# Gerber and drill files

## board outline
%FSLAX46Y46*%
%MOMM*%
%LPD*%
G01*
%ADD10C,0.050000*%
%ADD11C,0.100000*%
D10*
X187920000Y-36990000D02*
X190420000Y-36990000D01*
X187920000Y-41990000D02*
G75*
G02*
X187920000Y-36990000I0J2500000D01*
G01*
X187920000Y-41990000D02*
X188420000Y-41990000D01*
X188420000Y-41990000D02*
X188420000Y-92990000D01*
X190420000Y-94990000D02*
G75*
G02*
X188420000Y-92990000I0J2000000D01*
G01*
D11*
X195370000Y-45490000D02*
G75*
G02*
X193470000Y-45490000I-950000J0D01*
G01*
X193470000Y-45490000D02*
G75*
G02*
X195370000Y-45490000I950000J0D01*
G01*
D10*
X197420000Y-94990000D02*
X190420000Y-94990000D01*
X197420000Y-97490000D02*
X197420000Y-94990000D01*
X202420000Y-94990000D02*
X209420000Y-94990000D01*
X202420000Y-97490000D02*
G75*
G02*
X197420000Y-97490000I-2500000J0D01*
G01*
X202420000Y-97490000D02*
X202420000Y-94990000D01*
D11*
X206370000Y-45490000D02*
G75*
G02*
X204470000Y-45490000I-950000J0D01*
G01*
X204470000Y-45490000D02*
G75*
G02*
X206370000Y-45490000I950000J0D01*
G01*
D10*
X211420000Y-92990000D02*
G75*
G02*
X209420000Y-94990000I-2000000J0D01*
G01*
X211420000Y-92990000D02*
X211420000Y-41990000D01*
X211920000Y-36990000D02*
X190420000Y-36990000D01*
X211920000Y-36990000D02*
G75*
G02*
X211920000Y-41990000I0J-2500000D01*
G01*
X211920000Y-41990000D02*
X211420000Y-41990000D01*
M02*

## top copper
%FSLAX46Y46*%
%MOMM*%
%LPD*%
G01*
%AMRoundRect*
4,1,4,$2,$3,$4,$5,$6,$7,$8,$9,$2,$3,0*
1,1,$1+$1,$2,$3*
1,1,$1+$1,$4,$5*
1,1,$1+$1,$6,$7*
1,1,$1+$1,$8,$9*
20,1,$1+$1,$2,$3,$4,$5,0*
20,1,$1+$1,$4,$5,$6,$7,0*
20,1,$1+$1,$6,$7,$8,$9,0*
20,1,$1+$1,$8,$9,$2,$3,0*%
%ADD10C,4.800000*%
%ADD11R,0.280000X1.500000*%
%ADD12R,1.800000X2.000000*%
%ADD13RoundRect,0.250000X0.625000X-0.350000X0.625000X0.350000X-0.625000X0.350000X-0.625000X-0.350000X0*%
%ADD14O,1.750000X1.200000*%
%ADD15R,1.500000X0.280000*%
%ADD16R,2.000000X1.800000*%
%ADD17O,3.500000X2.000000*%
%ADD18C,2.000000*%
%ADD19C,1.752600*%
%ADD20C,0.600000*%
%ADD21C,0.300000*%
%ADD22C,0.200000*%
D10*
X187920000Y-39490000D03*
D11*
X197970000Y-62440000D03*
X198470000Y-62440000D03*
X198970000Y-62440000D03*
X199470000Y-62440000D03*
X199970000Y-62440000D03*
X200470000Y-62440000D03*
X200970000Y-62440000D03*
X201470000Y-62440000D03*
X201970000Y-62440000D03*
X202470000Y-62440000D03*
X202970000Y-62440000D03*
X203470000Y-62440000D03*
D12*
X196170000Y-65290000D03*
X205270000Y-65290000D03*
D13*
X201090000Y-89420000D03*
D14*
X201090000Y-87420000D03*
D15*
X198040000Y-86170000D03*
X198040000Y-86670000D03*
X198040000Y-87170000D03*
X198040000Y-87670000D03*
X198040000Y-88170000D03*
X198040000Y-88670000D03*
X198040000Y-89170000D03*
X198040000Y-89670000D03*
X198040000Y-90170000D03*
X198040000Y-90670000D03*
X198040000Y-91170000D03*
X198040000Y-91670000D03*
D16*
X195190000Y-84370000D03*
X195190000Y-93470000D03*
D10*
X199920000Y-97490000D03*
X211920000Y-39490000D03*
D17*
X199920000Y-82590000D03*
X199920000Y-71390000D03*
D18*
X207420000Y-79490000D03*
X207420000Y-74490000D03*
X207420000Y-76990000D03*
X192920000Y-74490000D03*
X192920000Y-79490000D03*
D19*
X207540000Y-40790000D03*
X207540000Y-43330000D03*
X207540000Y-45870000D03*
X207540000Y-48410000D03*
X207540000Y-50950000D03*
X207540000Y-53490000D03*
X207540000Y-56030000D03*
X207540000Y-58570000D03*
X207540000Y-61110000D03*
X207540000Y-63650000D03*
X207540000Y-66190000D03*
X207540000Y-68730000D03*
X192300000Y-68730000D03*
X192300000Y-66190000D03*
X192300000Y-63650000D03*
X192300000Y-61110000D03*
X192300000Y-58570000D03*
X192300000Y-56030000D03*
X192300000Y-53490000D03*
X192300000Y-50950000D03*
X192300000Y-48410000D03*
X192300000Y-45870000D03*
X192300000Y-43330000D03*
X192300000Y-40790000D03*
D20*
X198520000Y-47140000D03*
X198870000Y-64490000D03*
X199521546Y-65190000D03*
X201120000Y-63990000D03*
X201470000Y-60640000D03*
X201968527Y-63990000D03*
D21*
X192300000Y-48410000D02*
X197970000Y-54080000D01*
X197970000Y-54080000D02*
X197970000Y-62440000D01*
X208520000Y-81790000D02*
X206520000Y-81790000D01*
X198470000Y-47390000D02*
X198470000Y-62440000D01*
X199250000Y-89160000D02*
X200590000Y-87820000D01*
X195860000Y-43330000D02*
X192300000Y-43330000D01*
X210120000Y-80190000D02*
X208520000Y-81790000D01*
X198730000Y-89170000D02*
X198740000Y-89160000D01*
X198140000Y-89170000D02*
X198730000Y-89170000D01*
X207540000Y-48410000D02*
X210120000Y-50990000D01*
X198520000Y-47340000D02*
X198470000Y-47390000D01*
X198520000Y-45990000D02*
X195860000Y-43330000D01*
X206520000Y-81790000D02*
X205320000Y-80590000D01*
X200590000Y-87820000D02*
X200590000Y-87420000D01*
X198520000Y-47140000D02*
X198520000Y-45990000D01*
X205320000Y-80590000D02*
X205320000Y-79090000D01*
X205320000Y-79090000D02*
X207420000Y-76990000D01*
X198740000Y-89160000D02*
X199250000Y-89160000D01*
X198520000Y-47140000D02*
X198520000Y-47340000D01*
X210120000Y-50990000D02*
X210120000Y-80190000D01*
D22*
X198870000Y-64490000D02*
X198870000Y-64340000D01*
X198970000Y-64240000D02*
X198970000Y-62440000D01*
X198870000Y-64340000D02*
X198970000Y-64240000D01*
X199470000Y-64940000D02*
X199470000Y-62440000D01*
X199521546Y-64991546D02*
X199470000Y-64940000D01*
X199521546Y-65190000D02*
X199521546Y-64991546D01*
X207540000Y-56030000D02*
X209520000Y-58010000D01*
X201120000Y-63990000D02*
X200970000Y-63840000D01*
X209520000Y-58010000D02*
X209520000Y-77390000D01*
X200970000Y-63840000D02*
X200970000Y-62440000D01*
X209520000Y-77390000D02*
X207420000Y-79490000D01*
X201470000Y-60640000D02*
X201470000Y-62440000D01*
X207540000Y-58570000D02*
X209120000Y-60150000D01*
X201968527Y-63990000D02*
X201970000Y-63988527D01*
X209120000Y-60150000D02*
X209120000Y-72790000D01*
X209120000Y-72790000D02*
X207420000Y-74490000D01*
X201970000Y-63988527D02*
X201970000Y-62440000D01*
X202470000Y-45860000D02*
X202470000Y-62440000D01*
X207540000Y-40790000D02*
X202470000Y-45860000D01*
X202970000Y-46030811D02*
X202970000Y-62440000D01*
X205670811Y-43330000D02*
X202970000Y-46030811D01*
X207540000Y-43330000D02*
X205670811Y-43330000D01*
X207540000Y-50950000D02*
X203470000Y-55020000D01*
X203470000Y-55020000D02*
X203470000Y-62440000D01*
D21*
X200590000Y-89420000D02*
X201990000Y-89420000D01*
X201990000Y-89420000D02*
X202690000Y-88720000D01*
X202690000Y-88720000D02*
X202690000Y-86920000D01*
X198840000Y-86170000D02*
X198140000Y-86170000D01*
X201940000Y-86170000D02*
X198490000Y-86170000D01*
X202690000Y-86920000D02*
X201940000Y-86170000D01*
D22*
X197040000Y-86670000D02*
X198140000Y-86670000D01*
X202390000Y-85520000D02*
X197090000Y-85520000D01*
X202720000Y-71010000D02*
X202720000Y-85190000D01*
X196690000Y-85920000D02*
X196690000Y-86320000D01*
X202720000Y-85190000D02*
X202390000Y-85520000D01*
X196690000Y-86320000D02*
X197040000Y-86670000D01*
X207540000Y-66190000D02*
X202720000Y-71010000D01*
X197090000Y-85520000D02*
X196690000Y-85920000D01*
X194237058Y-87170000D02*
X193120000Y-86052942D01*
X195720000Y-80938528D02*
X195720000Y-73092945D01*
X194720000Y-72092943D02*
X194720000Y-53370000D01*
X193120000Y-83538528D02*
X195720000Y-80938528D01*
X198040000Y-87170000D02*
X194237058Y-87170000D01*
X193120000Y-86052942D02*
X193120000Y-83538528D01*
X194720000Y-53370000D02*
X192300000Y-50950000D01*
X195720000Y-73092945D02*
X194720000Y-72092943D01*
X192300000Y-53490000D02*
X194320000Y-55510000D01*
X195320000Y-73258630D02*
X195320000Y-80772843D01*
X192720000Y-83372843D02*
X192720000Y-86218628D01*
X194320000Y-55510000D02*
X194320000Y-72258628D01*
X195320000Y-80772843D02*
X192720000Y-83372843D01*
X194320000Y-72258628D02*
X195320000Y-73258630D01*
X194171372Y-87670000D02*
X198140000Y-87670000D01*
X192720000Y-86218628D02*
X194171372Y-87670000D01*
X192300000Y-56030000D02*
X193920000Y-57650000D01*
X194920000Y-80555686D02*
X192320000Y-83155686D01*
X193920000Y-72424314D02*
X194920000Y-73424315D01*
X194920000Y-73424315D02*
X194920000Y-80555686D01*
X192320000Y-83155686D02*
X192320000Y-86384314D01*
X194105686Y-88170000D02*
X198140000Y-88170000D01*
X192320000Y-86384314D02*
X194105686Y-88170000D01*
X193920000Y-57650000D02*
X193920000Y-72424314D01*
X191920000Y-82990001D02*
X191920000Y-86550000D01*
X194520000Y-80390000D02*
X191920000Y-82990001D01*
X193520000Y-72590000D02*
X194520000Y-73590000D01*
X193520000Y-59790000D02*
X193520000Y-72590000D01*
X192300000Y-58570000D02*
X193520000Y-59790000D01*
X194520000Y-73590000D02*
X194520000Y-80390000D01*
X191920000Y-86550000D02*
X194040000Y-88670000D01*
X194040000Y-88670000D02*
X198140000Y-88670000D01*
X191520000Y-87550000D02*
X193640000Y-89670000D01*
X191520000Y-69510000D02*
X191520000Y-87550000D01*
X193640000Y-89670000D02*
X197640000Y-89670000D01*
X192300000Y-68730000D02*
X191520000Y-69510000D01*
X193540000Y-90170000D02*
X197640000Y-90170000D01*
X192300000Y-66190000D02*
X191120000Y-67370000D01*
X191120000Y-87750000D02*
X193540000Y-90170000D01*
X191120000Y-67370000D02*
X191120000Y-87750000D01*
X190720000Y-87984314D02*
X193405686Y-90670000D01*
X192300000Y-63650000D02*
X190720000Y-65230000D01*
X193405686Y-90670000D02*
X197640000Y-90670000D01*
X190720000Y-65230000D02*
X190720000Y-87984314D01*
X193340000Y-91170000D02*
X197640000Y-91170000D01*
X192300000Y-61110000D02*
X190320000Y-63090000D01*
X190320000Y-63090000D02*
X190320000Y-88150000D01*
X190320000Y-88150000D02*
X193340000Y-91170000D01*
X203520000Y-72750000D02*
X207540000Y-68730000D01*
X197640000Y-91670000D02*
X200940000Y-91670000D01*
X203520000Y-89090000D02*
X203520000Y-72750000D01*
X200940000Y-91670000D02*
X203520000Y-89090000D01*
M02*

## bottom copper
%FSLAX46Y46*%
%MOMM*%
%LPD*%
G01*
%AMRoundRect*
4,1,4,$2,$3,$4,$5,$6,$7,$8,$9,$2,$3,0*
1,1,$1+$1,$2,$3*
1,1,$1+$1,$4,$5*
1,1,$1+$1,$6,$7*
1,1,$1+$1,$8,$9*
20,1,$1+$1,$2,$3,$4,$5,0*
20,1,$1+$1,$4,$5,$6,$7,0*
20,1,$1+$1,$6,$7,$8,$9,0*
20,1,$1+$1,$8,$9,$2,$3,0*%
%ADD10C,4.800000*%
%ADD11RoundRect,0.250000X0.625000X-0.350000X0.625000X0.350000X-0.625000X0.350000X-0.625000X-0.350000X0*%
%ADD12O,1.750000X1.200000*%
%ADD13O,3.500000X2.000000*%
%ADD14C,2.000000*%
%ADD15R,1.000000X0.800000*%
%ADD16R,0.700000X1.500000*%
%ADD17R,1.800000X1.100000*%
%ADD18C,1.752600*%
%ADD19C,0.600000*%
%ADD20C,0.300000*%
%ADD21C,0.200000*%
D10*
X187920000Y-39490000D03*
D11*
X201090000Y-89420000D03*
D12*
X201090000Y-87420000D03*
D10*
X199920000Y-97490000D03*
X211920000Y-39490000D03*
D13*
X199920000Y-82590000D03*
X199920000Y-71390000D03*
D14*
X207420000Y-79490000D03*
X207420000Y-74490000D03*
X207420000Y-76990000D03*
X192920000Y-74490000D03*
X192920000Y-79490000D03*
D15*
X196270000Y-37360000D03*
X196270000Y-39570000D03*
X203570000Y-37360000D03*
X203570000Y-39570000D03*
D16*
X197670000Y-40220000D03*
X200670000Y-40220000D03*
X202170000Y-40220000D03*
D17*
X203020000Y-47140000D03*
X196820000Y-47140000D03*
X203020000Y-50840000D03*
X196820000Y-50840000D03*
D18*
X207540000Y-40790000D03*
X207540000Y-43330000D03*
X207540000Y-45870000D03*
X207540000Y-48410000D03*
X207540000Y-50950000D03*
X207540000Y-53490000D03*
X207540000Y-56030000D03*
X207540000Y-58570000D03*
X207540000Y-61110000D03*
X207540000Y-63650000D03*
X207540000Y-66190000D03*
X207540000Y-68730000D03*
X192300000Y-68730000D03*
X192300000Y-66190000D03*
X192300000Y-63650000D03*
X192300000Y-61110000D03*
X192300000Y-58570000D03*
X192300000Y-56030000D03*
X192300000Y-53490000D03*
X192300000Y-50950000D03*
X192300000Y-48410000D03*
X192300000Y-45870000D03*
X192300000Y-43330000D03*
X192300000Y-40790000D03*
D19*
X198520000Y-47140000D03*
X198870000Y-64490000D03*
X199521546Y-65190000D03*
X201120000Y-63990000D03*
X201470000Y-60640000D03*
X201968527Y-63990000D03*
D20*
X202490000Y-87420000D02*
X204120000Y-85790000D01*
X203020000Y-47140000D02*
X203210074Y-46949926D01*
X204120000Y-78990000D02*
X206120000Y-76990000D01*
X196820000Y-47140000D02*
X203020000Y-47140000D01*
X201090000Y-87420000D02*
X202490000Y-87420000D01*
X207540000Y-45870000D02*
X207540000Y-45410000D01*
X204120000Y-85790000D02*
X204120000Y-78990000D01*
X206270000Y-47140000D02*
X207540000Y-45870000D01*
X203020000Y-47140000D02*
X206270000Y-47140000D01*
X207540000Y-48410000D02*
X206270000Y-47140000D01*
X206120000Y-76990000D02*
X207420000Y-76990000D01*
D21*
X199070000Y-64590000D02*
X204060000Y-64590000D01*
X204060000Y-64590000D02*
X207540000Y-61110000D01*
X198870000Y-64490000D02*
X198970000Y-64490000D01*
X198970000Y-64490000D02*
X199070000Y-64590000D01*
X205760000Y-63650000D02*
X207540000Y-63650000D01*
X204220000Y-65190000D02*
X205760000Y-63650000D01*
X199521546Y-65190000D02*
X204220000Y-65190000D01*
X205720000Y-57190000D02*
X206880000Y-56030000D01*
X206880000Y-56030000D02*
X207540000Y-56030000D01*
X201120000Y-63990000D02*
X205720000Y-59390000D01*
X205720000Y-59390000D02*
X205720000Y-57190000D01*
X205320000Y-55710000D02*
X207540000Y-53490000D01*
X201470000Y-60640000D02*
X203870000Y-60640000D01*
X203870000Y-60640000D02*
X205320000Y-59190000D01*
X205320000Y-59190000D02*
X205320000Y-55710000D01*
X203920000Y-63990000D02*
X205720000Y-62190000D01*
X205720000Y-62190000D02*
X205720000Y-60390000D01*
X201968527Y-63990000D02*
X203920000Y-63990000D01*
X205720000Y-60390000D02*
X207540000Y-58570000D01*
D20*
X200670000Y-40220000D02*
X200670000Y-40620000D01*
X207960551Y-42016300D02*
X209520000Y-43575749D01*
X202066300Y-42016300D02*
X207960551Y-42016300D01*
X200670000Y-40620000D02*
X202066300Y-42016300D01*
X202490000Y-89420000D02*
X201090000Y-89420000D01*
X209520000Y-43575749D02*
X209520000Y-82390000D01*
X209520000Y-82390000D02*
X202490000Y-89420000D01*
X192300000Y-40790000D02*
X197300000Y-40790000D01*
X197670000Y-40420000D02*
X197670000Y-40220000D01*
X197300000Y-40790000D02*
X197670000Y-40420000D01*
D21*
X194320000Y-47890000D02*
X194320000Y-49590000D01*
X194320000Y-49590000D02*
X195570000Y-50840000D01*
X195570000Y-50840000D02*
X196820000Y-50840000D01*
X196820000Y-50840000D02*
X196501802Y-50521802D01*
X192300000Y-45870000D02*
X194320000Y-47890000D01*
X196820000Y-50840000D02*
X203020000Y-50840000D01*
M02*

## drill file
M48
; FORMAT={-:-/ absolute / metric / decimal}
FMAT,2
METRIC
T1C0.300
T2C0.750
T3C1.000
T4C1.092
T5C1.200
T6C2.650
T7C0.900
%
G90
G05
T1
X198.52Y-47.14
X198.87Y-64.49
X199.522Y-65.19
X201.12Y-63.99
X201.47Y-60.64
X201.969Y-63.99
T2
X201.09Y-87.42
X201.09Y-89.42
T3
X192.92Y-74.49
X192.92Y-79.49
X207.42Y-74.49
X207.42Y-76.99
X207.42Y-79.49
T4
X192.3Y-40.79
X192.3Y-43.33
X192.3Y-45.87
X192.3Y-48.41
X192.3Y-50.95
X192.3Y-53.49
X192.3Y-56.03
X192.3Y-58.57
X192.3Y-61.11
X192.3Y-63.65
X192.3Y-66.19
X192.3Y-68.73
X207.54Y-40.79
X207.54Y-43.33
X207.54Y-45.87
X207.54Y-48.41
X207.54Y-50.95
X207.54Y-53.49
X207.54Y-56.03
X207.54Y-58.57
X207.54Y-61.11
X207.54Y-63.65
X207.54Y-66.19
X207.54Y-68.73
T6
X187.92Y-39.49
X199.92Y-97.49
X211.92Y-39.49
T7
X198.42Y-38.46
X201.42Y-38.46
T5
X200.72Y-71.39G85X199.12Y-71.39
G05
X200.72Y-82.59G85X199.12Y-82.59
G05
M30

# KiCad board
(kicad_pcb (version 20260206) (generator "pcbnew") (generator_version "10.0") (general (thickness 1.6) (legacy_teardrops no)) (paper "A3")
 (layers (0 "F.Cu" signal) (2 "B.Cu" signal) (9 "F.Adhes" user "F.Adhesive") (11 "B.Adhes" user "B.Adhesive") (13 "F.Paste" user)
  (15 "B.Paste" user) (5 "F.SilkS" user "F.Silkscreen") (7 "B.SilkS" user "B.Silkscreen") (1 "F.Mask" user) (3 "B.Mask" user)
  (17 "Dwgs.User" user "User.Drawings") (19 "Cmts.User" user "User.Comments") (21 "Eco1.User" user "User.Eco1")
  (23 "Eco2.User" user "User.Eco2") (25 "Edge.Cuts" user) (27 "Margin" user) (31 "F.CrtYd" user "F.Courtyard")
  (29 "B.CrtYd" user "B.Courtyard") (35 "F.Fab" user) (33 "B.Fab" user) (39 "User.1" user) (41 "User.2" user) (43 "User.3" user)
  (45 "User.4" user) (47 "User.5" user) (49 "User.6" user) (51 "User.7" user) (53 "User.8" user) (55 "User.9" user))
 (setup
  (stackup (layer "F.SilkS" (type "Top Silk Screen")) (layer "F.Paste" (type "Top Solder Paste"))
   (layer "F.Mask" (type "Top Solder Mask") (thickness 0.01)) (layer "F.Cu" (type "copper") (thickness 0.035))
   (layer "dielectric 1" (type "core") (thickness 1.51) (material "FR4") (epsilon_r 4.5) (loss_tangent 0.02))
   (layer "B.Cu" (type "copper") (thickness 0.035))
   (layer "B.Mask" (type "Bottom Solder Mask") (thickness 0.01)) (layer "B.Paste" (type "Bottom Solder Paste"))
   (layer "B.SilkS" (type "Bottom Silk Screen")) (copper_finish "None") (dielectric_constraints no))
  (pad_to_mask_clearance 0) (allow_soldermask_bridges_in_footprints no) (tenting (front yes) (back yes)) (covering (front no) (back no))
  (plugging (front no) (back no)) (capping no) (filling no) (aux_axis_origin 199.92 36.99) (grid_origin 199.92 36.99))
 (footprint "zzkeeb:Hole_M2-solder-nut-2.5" (layer "F.Cu") (at 187.92 39.49)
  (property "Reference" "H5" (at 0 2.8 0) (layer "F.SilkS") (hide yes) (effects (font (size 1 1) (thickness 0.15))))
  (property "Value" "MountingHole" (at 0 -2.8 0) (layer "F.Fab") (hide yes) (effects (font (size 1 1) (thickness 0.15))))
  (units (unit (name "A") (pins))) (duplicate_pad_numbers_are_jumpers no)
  (pad "" thru_hole circle (at 0 0) (size 4.8 4.8) (drill 2.65) (layers "*.Cu" "F.Mask") (remove_unused_layers no)))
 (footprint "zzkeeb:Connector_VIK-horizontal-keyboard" (layer "F.Cu") (at 200.72 63.99)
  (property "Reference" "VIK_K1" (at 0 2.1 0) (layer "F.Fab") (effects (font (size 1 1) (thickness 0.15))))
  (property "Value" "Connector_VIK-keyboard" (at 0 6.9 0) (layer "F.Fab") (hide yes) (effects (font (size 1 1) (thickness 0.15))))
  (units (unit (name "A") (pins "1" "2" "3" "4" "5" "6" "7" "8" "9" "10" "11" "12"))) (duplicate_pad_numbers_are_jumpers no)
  (pad "1" smd rect (at -2.75 -1.55) (size 0.28 1.5) (layers "F.Cu" "F.Mask" "F.Paste") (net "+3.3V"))
  (pad "2" smd rect (at -2.25 -1.55) (size 0.28 1.5) (layers "F.Cu" "F.Mask" "F.Paste") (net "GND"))
  (pad "3" smd rect (at -1.75 -1.55) (size 0.28 1.5) (layers "F.Cu" "F.Mask" "F.Paste") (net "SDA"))
  (pad "4" smd rect (at -1.25 -1.55) (size 0.28 1.5) (layers "F.Cu" "F.Mask" "F.Paste") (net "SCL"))
  (pad "5" smd rect (at -0.75 -1.55) (size 0.28 1.5) (layers "F.Cu" "F.Mask" "F.Paste") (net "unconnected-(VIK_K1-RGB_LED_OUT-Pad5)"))
  (pad "6" smd rect (at -0.25 -1.55) (size 0.28 1.5) (layers "F.Cu" "F.Mask" "F.Paste") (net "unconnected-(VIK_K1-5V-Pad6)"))
  (pad "7" smd rect (at 0.25 -1.55) (size 0.28 1.5) (layers "F.Cu" "F.Mask" "F.Paste") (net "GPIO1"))
  (pad "8" smd rect (at 0.75 -1.55) (size 0.28 1.5) (layers "F.Cu" "F.Mask" "F.Paste") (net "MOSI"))
  (pad "9" smd rect (at 1.25 -1.55) (size 0.28 1.5) (layers "F.Cu" "F.Mask" "F.Paste") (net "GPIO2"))
  (pad "10" smd rect (at 1.75 -1.55) (size 0.28 1.5) (layers "F.Cu" "F.Mask" "F.Paste") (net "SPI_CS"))
  (pad "11" smd rect (at 2.25 -1.55) (size 0.28 1.5) (layers "F.Cu" "F.Mask" "F.Paste") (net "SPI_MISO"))
  (pad "12" smd rect (at 2.75 -1.55) (size 0.28 1.5) (layers "F.Cu" "F.Mask" "F.Paste") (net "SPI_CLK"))
  (pad "MP" smd rect (at -4.55 1.3) (size 1.8 2) (layers "F.Cu" "F.Mask" "F.Paste"))
  (pad "MP" smd rect (at 4.55 1.3) (size 1.8 2) (layers "F.Cu" "F.Mask" "F.Paste")))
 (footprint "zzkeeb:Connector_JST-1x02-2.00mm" (layer "F.Cu") (at 201.09 89.42 90)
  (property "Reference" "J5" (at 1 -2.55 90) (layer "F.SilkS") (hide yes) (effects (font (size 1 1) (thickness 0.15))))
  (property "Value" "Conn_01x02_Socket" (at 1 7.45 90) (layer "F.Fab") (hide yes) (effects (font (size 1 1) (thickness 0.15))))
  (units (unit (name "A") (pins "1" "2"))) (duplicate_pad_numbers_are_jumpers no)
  (pad "1" thru_hole roundrect (at 0 0 90) (size 1.2 1.75) (drill 0.75) (layers "*.Cu" "*.Mask") (remove_unused_layers no)
   (roundrect_rratio 0.208333) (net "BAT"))
  (pad "2" thru_hole oval (at 2 0 90) (size 1.2 1.75) (drill 0.75) (layers "*.Cu" "*.Mask") (remove_unused_layers no) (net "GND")))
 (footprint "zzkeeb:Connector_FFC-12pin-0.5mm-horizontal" (layer "F.Cu") (at 196.49 88.92 -90)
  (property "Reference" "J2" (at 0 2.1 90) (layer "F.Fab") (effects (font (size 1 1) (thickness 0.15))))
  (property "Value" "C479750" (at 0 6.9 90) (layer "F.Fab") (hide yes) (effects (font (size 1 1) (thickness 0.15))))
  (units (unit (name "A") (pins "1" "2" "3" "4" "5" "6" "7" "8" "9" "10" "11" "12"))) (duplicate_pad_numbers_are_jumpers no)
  (pad "1" smd rect (at -2.75 -1.55 270) (size 0.28 1.5) (layers "F.Cu" "F.Mask" "F.Paste") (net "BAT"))
  (pad "2" smd rect (at -2.25 -1.55 270) (size 0.28 1.5) (layers "F.Cu" "F.Mask" "F.Paste") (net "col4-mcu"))
  (pad "3" smd rect (at -1.75 -1.55 270) (size 0.28 1.5) (layers "F.Cu" "F.Mask" "F.Paste") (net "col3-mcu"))
  (pad "4" smd rect (at -1.25 -1.55 270) (size 0.28 1.5) (layers "F.Cu" "F.Mask" "F.Paste") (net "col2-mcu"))
  (pad "5" smd rect (at -0.75 -1.55 270) (size 0.28 1.5) (layers "F.Cu" "F.Mask" "F.Paste") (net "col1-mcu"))
  (pad "6" smd rect (at -0.25 -1.55 270) (size 0.28 1.5) (layers "F.Cu" "F.Mask" "F.Paste") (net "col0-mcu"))
  (pad "7" smd rect (at 0.25 -1.55 270) (size 0.28 1.5) (layers "F.Cu" "F.Mask" "F.Paste") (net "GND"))
  (pad "8" smd rect (at 0.75 -1.55 270) (size 0.28 1.5) (layers "F.Cu" "F.Mask" "F.Paste") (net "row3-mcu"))
  (pad "9" smd rect (at 1.25 -1.55 270) (size 0.28 1.5) (layers "F.Cu" "F.Mask" "F.Paste") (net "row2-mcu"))
  (pad "10" smd rect (at 1.75 -1.55 270) (size 0.28 1.5) (layers "F.Cu" "F.Mask" "F.Paste") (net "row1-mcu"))
  (pad "11" smd rect (at 2.25 -1.55 270) (size 0.28 1.5) (layers "F.Cu" "F.Mask" "F.Paste") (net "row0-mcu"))
  (pad "12" smd rect (at 2.75 -1.55 270) (size 0.28 1.5) (layers "F.Cu" "F.Mask" "F.Paste") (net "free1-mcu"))
  (pad "MP" smd rect (at -4.55 1.3 270) (size 1.8 2) (layers "F.Cu" "F.Mask" "F.Paste"))
  (pad "MP" smd rect (at 4.55 1.3 270) (size 1.8 2) (layers "F.Cu" "F.Mask" "F.Paste")))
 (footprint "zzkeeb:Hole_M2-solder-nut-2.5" (layer "F.Cu") (at 199.92 97.49)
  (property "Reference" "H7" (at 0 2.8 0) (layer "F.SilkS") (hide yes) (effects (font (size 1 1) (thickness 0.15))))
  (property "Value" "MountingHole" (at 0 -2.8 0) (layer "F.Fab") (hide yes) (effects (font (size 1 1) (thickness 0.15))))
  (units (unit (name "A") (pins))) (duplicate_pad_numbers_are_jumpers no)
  (pad "" thru_hole circle (at 0 0) (size 4.8 4.8) (drill 2.65) (layers "*.Cu" "F.Mask") (remove_unused_layers no)))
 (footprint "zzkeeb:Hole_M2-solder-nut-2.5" (layer "F.Cu") (at 211.92 39.49)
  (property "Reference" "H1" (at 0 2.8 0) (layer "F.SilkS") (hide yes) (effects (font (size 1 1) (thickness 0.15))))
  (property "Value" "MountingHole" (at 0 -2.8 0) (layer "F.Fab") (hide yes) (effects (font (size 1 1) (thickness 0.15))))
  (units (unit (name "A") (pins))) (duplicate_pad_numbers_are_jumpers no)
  (pad "" thru_hole circle (at 0 0) (size 4.8 4.8) (drill 2.65) (layers "*.Cu" "F.Mask") (remove_unused_layers no)))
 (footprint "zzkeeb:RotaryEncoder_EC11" (layer "F.Cu") (at 199.92 76.99 180)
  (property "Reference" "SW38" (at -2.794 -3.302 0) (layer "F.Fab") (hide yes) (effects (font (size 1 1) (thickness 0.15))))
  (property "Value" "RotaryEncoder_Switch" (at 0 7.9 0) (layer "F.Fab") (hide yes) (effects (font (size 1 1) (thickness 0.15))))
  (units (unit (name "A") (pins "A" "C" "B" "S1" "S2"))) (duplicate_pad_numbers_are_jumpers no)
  (pad "" thru_hole oval (at 0 -5.6 180) (size 3.5 2) (drill oval 2.8 1.2) (layers "*.Cu" "*.Mask") (remove_unused_layers no))
  (pad "" thru_hole oval (at 0 5.6 180) (size 3.5 2) (drill oval 2.8 1.2) (layers "*.Cu" "*.Mask") (remove_unused_layers no))
  (pad "A" thru_hole circle (at -7.5 -2.5 180) (size 2 2) (drill 1) (layers "*.Cu" "B.Mask") (remove_unused_layers no) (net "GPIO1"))
  (pad "B" thru_hole circle (at -7.5 2.5 180) (size 2 2) (drill 1) (layers "*.Cu" "B.Mask") (remove_unused_layers no) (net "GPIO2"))
  (pad "C" thru_hole circle (at -7.5 0 180) (size 2 2) (drill 1) (layers "*.Cu" "B.Mask") (remove_unused_layers no) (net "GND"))
  (pad "S1" thru_hole circle (at 7 2.5 180) (size 2 2) (drill 1) (layers "*.Cu" "B.Mask") (remove_unused_layers no)
   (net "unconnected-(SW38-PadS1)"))
  (pad "S2" thru_hole circle (at 7 -2.5 180) (size 2 2) (drill 1) (layers "*.Cu" "B.Mask") (remove_unused_layers no)
   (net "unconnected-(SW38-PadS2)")))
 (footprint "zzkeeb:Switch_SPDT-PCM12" (layer "B.Cu") (at 199.92 38.79)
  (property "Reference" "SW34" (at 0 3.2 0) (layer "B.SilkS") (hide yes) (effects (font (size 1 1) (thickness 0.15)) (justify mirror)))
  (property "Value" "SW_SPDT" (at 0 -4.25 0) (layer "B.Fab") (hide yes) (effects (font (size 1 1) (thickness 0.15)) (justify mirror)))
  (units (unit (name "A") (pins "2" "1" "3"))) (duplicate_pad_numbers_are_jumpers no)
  (pad "" smd rect (at -3.65 -1.43) (size 1 0.8) (layers "B.Cu" "B.Mask" "B.Paste"))
  (pad "" smd rect (at -3.65 0.78) (size 1 0.8) (layers "B.Cu" "B.Mask" "B.Paste"))
  (pad "" np_thru_hole circle (at -1.5 -0.33) (size 0.9 0.9) (drill 0.9) (layers "*.Cu" "*.Mask"))
  (pad "" np_thru_hole circle (at 1.5 -0.33) (size 0.9 0.9) (drill 0.9) (layers "*.Cu" "*.Mask"))
  (pad "" smd rect (at 3.65 -1.43) (size 1 0.8) (layers "B.Cu" "B.Mask" "B.Paste"))
  (pad "" smd rect (at 3.65 0.78) (size 1 0.8) (layers "B.Cu" "B.Mask" "B.Paste"))
  (pad "1" smd rect (at -2.25 1.43) (size 0.7 1.5) (layers "B.Cu" "B.Mask" "B.Paste") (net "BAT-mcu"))
  (pad "2" smd rect (at 0.75 1.43) (size 0.7 1.5) (layers "B.Cu" "B.Mask" "B.Paste") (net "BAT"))
  (pad "3" smd rect (at 2.25 1.43) (size 0.7 1.5) (layers "B.Cu" "B.Mask" "B.Paste") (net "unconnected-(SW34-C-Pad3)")))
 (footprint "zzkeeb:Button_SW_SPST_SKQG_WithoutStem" (layer "B.Cu") (at 199.92 48.99 180)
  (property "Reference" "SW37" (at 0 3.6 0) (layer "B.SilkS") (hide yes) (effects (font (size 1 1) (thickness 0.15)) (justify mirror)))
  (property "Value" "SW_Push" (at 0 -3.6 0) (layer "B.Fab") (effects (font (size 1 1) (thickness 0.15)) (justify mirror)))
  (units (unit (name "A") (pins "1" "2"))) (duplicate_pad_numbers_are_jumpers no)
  (pad "1" smd rect (at -3.1 1.85 180) (size 1.8 1.1) (layers "B.Cu" "B.Mask" "B.Paste") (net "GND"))
  (pad "1" smd rect (at 3.1 1.85 180) (size 1.8 1.1) (layers "B.Cu" "B.Mask" "B.Paste") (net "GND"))
  (pad "2" smd rect (at -3.1 -1.85 180) (size 1.8 1.1) (layers "B.Cu" "B.Mask" "B.Paste") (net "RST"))
  (pad "2" smd rect (at 3.1 -1.85 180) (size 1.8 1.1) (layers "B.Cu" "B.Mask" "B.Paste") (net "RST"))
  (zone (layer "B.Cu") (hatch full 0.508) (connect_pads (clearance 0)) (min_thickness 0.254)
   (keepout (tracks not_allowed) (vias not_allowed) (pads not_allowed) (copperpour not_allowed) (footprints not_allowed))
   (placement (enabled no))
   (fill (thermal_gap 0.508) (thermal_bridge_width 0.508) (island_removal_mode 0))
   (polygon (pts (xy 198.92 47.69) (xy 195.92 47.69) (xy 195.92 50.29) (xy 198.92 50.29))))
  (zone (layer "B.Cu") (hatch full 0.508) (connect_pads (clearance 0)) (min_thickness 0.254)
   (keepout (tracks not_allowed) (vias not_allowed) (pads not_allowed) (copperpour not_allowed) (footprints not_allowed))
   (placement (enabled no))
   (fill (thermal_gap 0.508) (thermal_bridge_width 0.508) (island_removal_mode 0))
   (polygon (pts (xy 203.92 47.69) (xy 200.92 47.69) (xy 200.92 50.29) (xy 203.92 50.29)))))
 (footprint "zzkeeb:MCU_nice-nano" (layer "B.Cu") (at 199.92 53.49 180)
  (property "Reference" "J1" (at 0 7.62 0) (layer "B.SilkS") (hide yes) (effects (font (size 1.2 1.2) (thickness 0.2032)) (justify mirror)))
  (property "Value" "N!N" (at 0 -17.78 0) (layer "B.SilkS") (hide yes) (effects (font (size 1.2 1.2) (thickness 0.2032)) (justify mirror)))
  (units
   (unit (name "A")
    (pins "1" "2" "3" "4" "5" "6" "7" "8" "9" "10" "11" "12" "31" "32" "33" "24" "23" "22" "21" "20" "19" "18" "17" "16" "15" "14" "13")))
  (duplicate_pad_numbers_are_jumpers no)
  (pad "1" thru_hole circle (at -7.62 12.7 270) (size 1.7526 1.7526) (drill 1.0922) (layers "*.Cu" "*.Mask") (remove_unused_layers no)
   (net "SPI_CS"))
  (pad "2" thru_hole circle (at -7.62 10.16 270) (size 1.7526 1.7526) (drill 1.0922) (layers "*.Cu" "*.Mask") (remove_unused_layers no)
   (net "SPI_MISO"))
  (pad "3" thru_hole circle (at -7.62 7.62 270) (size 1.7526 1.7526) (drill 1.0922) (layers "*.Cu" "*.Mask") (remove_unused_layers no)
   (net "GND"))
  (pad "4" thru_hole circle (at -7.62 5.08 270) (size 1.7526 1.7526) (drill 1.0922) (layers "*.Cu" "*.Mask") (remove_unused_layers no)
   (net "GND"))
  (pad "5" thru_hole circle (at -7.62 2.54 270) (size 1.7526 1.7526) (drill 1.0922) (layers "*.Cu" "*.Mask") (remove_unused_layers no)
   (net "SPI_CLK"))
  (pad "6" thru_hole circle (at -7.62 0 270) (size 1.7526 1.7526) (drill 1.0922) (layers "*.Cu" "*.Mask") (remove_unused_layers no)
   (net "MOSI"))
  (pad "7" thru_hole circle (at -7.62 -2.54 270) (size 1.7526 1.7526) (drill 1.0922) (layers "*.Cu" "*.Mask") (remove_unused_layers no)
   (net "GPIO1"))
  (pad "8" thru_hole circle (at -7.62 -5.08 270) (size 1.7526 1.7526) (drill 1.0922) (layers "*.Cu" "*.Mask") (remove_unused_layers no)
   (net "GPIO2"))
  (pad "9" thru_hole circle (at -7.62 -7.62 270) (size 1.7526 1.7526) (drill 1.0922) (layers "*.Cu" "*.Mask") (remove_unused_layers no)
   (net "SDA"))
  (pad "10" thru_hole circle (at -7.62 -10.16 270) (size 1.7526 1.7526) (drill 1.0922) (layers "*.Cu" "*.Mask") (remove_unused_layers no)
   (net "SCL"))
  (pad "11" thru_hole circle (at -7.62 -12.7 270) (size 1.7526 1.7526) (drill 1.0922) (layers "*.Cu" "*.Mask") (remove_unused_layers no)
   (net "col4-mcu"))
  (pad "12" thru_hole circle (at -7.62 -15.24 270) (size 1.7526 1.7526) (drill 1.0922) (layers "*.Cu" "*.Mask") (remove_unused_layers no)
   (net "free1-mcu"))
  (pad "13" thru_hole circle (at 7.62 -15.24 270) (size 1.7526 1.7526) (drill 1.0922) (layers "*.Cu" "*.Mask") (remove_unused_layers no)
   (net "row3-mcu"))
  (pad "14" thru_hole circle (at 7.62 -12.7 270) (size 1.7526 1.7526) (drill 1.0922) (layers "*.Cu" "*.Mask") (remove_unused_layers no)
   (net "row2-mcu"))
  (pad "15" thru_hole circle (at 7.62 -10.16 270) (size 1.7526 1.7526) (drill 1.0922) (layers "*.Cu" "*.Mask") (remove_unused_layers no)
   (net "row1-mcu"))
  (pad "16" thru_hole circle (at 7.62 -7.62 270) (size 1.7526 1.7526) (drill 1.0922) (layers "*.Cu" "*.Mask") (remove_unused_layers no)
   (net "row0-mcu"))
  (pad "17" thru_hole circle (at 7.62 -5.08 270) (size 1.7526 1.7526) (drill 1.0922) (layers "*.Cu" "*.Mask") (remove_unused_layers no)
   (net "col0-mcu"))
  (pad "18" thru_hole circle (at 7.62 -2.54 270) (size 1.7526 1.7526) (drill 1.0922) (layers "*.Cu" "*.Mask") (remove_unused_layers no)
   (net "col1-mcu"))
  (pad "19" thru_hole circle (at 7.62 0 270) (size 1.7526 1.7526) (drill 1.0922) (layers "*.Cu" "*.Mask") (remove_unused_layers no)
   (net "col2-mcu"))
  (pad "20" thru_hole circle (at 7.62 2.54 270) (size 1.7526 1.7526) (drill 1.0922) (layers "*.Cu" "*.Mask") (remove_unused_layers no)
   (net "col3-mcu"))
  (pad "21" thru_hole circle (at 7.62 5.08 270) (size 1.7526 1.7526) (drill 1.0922) (layers "*.Cu" "*.Mask") (remove_unused_layers no)
   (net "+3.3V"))
  (pad "22" thru_hole circle (at 7.62 7.62 270) (size 1.7526 1.7526) (drill 1.0922) (layers "*.Cu" "*.Mask") (remove_unused_layers no)
   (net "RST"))
  (pad "23" thru_hole circle (at 7.62 10.16 270) (size 1.7526 1.7526) (drill 1.0922) (layers "*.Cu" "*.Mask") (remove_unused_layers no)
   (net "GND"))
  (pad "24" thru_hole circle (at 7.62 12.7 270) (size 1.7526 1.7526) (drill 1.0922) (layers "*.Cu" "*.Mask") (remove_unused_layers no)
   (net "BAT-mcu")))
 (gr_line (start 187.92 36.99) (end 190.42 36.99) (stroke (width 0.05) (type default)) (layer "Edge.Cuts"))
 (gr_arc (start 187.92 41.99) (mid 185.42 39.49) (end 187.92 36.99) (stroke (width 0.05) (type default)) (layer "Edge.Cuts"))
 (gr_line (start 187.92 41.99) (end 188.42 41.99) (stroke (width 0.05) (type default)) (layer "Edge.Cuts"))
 (gr_line (start 188.42 41.99) (end 188.42 92.99) (stroke (width 0.05) (type default)) (layer "Edge.Cuts"))
 (gr_arc (start 190.42 94.99) (mid 189.005786 94.404214) (end 188.42 92.99) (stroke (width 0.05) (type default)) (layer "Edge.Cuts"))
 (gr_circle (center 194.42 45.49) (end 193.47 45.49) (stroke (width 0.1) (type default)) (fill no) (layer "Edge.Cuts"))
 (gr_line (start 197.42 94.99) (end 190.42 94.99) (stroke (width 0.05) (type default)) (layer "Edge.Cuts"))
 (gr_line (start 197.42 97.49) (end 197.42 94.99) (stroke (width 0.05) (type default)) (layer "Edge.Cuts"))
 (gr_line (start 202.42 94.99) (end 209.42 94.99) (stroke (width 0.05) (type default)) (layer "Edge.Cuts"))
 (gr_arc (start 202.42 97.49) (mid 199.92 99.99) (end 197.42 97.49) (stroke (width 0.05) (type default)) (layer "Edge.Cuts"))
 (gr_line (start 202.42 97.49) (end 202.42 94.99) (stroke (width 0.05) (type default)) (layer "Edge.Cuts"))
 (gr_circle (center 205.42 45.49) (end 204.47 45.49) (stroke (width 0.1) (type default)) (fill no) (layer "Edge.Cuts"))
 (gr_arc (start 211.42 92.99) (mid 210.834214 94.404214) (end 209.42 94.99) (stroke (width 0.05) (type default)) (layer "Edge.Cuts"))
 (gr_line (start 211.42 92.99) (end 211.42 41.99) (stroke (width 0.05) (type default)) (layer "Edge.Cuts"))
 (gr_line (start 211.92 36.99) (end 190.42 36.99) (stroke (width 0.05) (type default)) (layer "Edge.Cuts"))
 (gr_arc (start 211.92 36.99) (mid 214.42 39.49) (end 211.92 41.99) (stroke (width 0.05) (type default)) (layer "Edge.Cuts"))
 (gr_line (start 211.92 41.99) (end 211.42 41.99) (stroke (width 0.05) (type default)) (layer "Edge.Cuts"))
 (segment (start 192.3 48.41) (end 197.97 54.08) (width 0.3) (layer "F.Cu") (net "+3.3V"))
 (segment (start 197.97 54.08) (end 197.97 62.44) (width 0.3) (layer "F.Cu") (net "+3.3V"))
 (segment (start 208.52 81.79) (end 206.52 81.79) (width 0.3) (layer "F.Cu") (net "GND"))
 (segment (start 198.47 47.39) (end 198.47 62.44) (width 0.3) (layer "F.Cu") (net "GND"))
 (segment (start 199.25 89.16) (end 200.59 87.82) (width 0.3) (layer "F.Cu") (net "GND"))
 (segment (start 195.86 43.33) (end 192.3 43.33) (width 0.3) (layer "F.Cu") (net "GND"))
 (segment (start 210.12 80.19) (end 208.52 81.79) (width 0.3) (layer "F.Cu") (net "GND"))
 (segment (start 198.73 89.17) (end 198.74 89.16) (width 0.3) (layer "F.Cu") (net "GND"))
 (segment (start 198.14 89.17) (end 198.73 89.17) (width 0.3) (layer "F.Cu") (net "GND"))
 (segment (start 207.54 48.41) (end 210.12 50.99) (width 0.3) (layer "F.Cu") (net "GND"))
 (segment (start 198.52 47.34) (end 198.47 47.39) (width 0.3) (layer "F.Cu") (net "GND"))
 (segment (start 198.52 45.99) (end 195.86 43.33) (width 0.3) (layer "F.Cu") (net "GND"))
 (segment (start 206.52 81.79) (end 205.32 80.59) (width 0.3) (layer "F.Cu") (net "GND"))
 (segment (start 200.59 87.82) (end 200.59 87.42) (width 0.3) (layer "F.Cu") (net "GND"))
 (segment (start 198.52 47.14) (end 198.52 45.99) (width 0.3) (layer "F.Cu") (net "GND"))
 (segment (start 205.32 80.59) (end 205.32 79.09) (width 0.3) (layer "F.Cu") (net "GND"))
 (segment (start 205.32 79.09) (end 207.42 76.99) (width 0.3) (layer "F.Cu") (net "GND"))
 (segment (start 198.74 89.16) (end 199.25 89.16) (width 0.3) (layer "F.Cu") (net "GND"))
 (segment (start 198.52 47.14) (end 198.52 47.34) (width 0.3) (layer "F.Cu") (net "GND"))
 (segment (start 210.12 50.99) (end 210.12 80.19) (width 0.3) (layer "F.Cu") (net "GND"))
 (via (at 198.52 47.14) (size 0.6) (drill 0.3) (layers "F.Cu" "B.Cu") (capping no) (covering (front no) (back no))
  (plugging (front no) (back no)) (filling no) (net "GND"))
 (segment (start 202.49 87.42) (end 204.12 85.79) (width 0.3) (layer "B.Cu") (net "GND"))
 (segment (start 203.02 47.14) (end 203.210074 46.949926) (width 0.3) (layer "B.Cu") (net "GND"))
 (segment (start 204.12 78.99) (end 206.12 76.99) (width 0.3) (layer "B.Cu") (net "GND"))
 (segment (start 196.82 47.14) (end 203.02 47.14) (width 0.3) (layer "B.Cu") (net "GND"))
 (segment (start 201.09 87.42) (end 202.49 87.42) (width 0.3) (layer "B.Cu") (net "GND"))
 (segment (start 207.54 45.87) (end 207.54 45.41) (width 0.3) (layer "B.Cu") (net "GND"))
 (segment (start 204.12 85.79) (end 204.12 78.99) (width 0.3) (layer "B.Cu") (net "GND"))
 (segment (start 206.27 47.14) (end 207.54 45.87) (width 0.3) (layer "B.Cu") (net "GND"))
 (segment (start 203.02 47.14) (end 206.27 47.14) (width 0.3) (layer "B.Cu") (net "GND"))
 (segment (start 207.54 48.41) (end 206.27 47.14) (width 0.3) (layer "B.Cu") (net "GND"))
 (segment (start 206.12 76.99) (end 207.42 76.99) (width 0.3) (layer "B.Cu") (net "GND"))
 (segment (start 198.87 64.49) (end 198.87 64.34) (width 0.2) (layer "F.Cu") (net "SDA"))
 (segment (start 198.97 64.24) (end 198.97 62.44) (width 0.2) (layer "F.Cu") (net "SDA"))
 (segment (start 198.87 64.34) (end 198.97 64.24) (width 0.2) (layer "F.Cu") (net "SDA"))
 (via (at 198.87 64.49) (size 0.6) (drill 0.3) (layers "F.Cu" "B.Cu") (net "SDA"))
 (segment (start 199.07 64.59) (end 204.06 64.59) (width 0.2) (layer "B.Cu") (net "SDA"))
 (segment (start 204.06 64.59) (end 207.54 61.11) (width 0.2) (layer "B.Cu") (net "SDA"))
 (segment (start 198.87 64.49) (end 198.97 64.49) (width 0.2) (layer "B.Cu") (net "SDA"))
 (segment (start 198.97 64.49) (end 199.07 64.59) (width 0.2) (layer "B.Cu") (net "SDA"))
 (segment (start 199.47 64.94) (end 199.47 62.44) (width 0.2) (layer "F.Cu") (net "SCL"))
 (segment (start 199.521546 64.991546) (end 199.47 64.94) (width 0.2) (layer "F.Cu") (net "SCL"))
 (segment (start 199.521546 65.19) (end 199.521546 64.991546) (width 0.2) (layer "F.Cu") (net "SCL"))
 (via (at 199.521546 65.19) (size 0.6) (drill 0.3) (layers "F.Cu" "B.Cu") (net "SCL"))
 (segment (start 205.76 63.65) (end 207.54 63.65) (width 0.2) (layer "B.Cu") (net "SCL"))
 (segment (start 204.22 65.19) (end 205.76 63.65) (width 0.2) (layer "B.Cu") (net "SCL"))
 (segment (start 199.521546 65.19) (end 204.22 65.19) (width 0.2) (layer "B.Cu") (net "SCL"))
 (segment (start 207.54 56.03) (end 209.52 58.01) (width 0.2) (layer "F.Cu") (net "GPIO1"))
 (segment (start 201.12 63.99) (end 200.97 63.84) (width 0.2) (layer "F.Cu") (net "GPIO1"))
 (segment (start 209.52 58.01) (end 209.52 77.39) (width 0.2) (layer "F.Cu") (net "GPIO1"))
 (segment (start 200.97 63.84) (end 200.97 62.44) (width 0.2) (layer "F.Cu") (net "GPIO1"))
 (segment (start 209.52 77.39) (end 207.42 79.49) (width 0.2) (layer "F.Cu") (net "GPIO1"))
 (via (at 201.12 63.99) (size 0.6) (drill 0.3) (layers "F.Cu" "B.Cu") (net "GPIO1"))
 (segment (start 205.72 57.19) (end 206.88 56.03) (width 0.2) (layer "B.Cu") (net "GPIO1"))
 (segment (start 206.88 56.03) (end 207.54 56.03) (width 0.2) (layer "B.Cu") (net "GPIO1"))
 (segment (start 201.12 63.99) (end 205.72 59.39) (width 0.2) (layer "B.Cu") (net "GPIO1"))
 (segment (start 205.72 59.39) (end 205.72 57.19) (width 0.2) (layer "B.Cu") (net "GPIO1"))
 (segment (start 201.47 60.64) (end 201.47 62.44) (width 0.2) (layer "F.Cu") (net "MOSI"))
 (via (at 201.47 60.64) (size 0.6) (drill 0.3) (layers "F.Cu" "B.Cu") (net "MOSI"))
 (segment (start 205.32 55.71) (end 207.54 53.49) (width 0.2) (layer "B.Cu") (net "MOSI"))
 (segment (start 201.47 60.64) (end 203.87 60.64) (width 0.2) (layer "B.Cu") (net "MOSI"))
 (segment (start 203.87 60.64) (end 205.32 59.19) (width 0.2) (layer "B.Cu") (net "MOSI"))
 (segment (start 205.32 59.19) (end 205.32 55.71) (width 0.2) (layer "B.Cu") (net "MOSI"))
 (segment (start 207.54 58.57) (end 209.12 60.15) (width 0.2) (layer "F.Cu") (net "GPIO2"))
 (segment (start 201.968527 63.99) (end 201.97 63.988527) (width 0.2) (layer "F.Cu") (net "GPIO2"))
 (segment (start 209.12 60.15) (end 209.12 72.79) (width 0.2) (layer "F.Cu") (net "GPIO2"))
 (segment (start 209.12 72.79) (end 207.42 74.49) (width 0.2) (layer "F.Cu") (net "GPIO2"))
 (segment (start 201.97 63.988527) (end 201.97 62.44) (width 0.2) (layer "F.Cu") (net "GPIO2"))
 (via (at 201.968527 63.99) (size 0.6) (drill 0.3) (layers "F.Cu" "B.Cu") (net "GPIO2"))
 (segment (start 203.92 63.99) (end 205.72 62.19) (width 0.2) (layer "B.Cu") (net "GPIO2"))
 (segment (start 205.72 62.19) (end 205.72 60.39) (width 0.2) (layer "B.Cu") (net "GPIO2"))
 (segment (start 201.968527 63.99) (end 203.92 63.99) (width 0.2) (layer "B.Cu") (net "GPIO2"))
 (segment (start 205.72 60.39) (end 207.54 58.57) (width 0.2) (layer "B.Cu") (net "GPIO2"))
 (segment (start 202.47 45.86) (end 202.47 62.44) (width 0.2) (layer "F.Cu") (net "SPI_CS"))
 (segment (start 207.54 40.79) (end 202.47 45.86) (width 0.2) (layer "F.Cu") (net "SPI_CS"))
 (segment (start 202.97 46.030811) (end 202.97 62.44) (width 0.2) (layer "F.Cu") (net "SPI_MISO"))
 (segment (start 205.670811 43.33) (end 202.97 46.030811) (width 0.2) (layer "F.Cu") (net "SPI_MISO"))
 (segment (start 207.54 43.33) (end 205.670811 43.33) (width 0.2) (layer "F.Cu") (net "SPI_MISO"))
 (segment (start 207.54 50.95) (end 203.47 55.02) (width 0.2) (layer "F.Cu") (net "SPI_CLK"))
 (segment (start 203.47 55.02) (end 203.47 62.44) (width 0.2) (layer "F.Cu") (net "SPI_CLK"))
 (segment (start 200.59 89.42) (end 201.99 89.42) (width 0.3) (layer "F.Cu") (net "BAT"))
 (segment (start 201.99 89.42) (end 202.69 88.72) (width 0.3) (layer "F.Cu") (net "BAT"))
 (segment (start 202.69 88.72) (end 202.69 86.92) (width 0.3) (layer "F.Cu") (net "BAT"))
 (segment (start 198.84 86.17) (end 198.14 86.17) (width 0.3) (layer "F.Cu") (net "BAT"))
 (segment (start 201.94 86.17) (end 198.49 86.17) (width 0.3) (layer "F.Cu") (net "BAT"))
 (segment (start 202.69 86.92) (end 201.94 86.17) (width 0.3) (layer "F.Cu") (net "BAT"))
 (segment (start 200.67 40.22) (end 200.67 40.62) (width 0.3) (layer "B.Cu") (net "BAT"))
 (segment (start 207.960551 42.0163) (end 209.52 43.575749) (width 0.3) (layer "B.Cu") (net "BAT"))
 (segment (start 202.0663 42.0163) (end 207.960551 42.0163) (width 0.3) (layer "B.Cu") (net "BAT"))
 (segment (start 200.67 40.62) (end 202.0663 42.0163) (width 0.3) (layer "B.Cu") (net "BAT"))
 (segment (start 202.49 89.42) (end 201.09 89.42) (width 0.3) (layer "B.Cu") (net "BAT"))
 (segment (start 209.52 43.575749) (end 209.52 82.39) (width 0.3) (layer "B.Cu") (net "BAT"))
 (segment (start 209.52 82.39) (end 202.49 89.42) (width 0.3) (layer "B.Cu") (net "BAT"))
 (segment (start 197.04 86.67) (end 198.14 86.67) (width 0.2) (layer "F.Cu") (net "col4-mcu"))
 (segment (start 202.39 85.52) (end 197.09 85.52) (width 0.2) (layer "F.Cu") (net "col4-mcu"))
 (segment (start 202.72 71.01) (end 202.72 85.19) (width 0.2) (layer "F.Cu") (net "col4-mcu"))
 (segment (start 196.69 85.92) (end 196.69 86.32) (width 0.2) (layer "F.Cu") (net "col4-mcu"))
 (segment (start 202.72 85.19) (end 202.39 85.52) (width 0.2) (layer "F.Cu") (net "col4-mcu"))
 (segment (start 196.69 86.32) (end 197.04 86.67) (width 0.2) (layer "F.Cu") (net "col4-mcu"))
 (segment (start 207.54 66.19) (end 202.72 71.01) (width 0.2) (layer "F.Cu") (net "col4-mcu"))
 (segment (start 197.09 85.52) (end 196.69 85.92) (width 0.2) (layer "F.Cu") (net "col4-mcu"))
 (segment (start 194.237058 87.17) (end 193.12 86.052942) (width 0.2) (layer "F.Cu") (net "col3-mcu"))
 (segment (start 195.72 80.938528) (end 195.72 73.092945) (width 0.2) (layer "F.Cu") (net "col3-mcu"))
 (segment (start 194.72 72.092943) (end 194.72 53.37) (width 0.2) (layer "F.Cu") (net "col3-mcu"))
 (segment (start 193.12 83.538528) (end 195.72 80.938528) (width 0.2) (layer "F.Cu") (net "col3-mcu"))
 (segment (start 198.04 87.17) (end 194.237058 87.17) (width 0.2) (layer "F.Cu") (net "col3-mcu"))
 (segment (start 193.12 86.052942) (end 193.12 83.538528) (width 0.2) (layer "F.Cu") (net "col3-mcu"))
 (segment (start 194.72 53.37) (end 192.3 50.95) (width 0.2) (layer "F.Cu") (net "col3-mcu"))
 (segment (start 195.72 73.092945) (end 194.72 72.092943) (width 0.2) (layer "F.Cu") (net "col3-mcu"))
 (segment (start 192.3 53.49) (end 194.32 55.51) (width 0.2) (layer "F.Cu") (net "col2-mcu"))
 (segment (start 195.32 73.25863) (end 195.32 80.772843) (width 0.2) (layer "F.Cu") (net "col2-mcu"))
 (segment (start 192.72 83.372843) (end 192.72 86.218628) (width 0.2) (layer "F.Cu") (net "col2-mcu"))
 (segment (start 194.32 55.51) (end 194.32 72.258628) (width 0.2) (layer "F.Cu") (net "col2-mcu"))
 (segment (start 195.32 80.772843) (end 192.72 83.372843) (width 0.2) (layer "F.Cu") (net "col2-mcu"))
 (segment (start 194.32 72.258628) (end 195.32 73.25863) (width 0.2) (layer "F.Cu") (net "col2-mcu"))
 (segment (start 194.171372 87.67) (end 198.14 87.67) (width 0.2) (layer "F.Cu") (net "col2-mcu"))
 (segment (start 192.72 86.218628) (end 194.171372 87.67) (width 0.2) (layer "F.Cu") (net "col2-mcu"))
 (segment (start 192.3 56.03) (end 193.92 57.65) (width 0.2) (layer "F.Cu") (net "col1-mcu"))
 (segment (start 194.92 80.555686) (end 192.32 83.155686) (width 0.2) (layer "F.Cu") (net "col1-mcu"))
 (segment (start 193.92 72.424314) (end 194.92 73.424315) (width 0.2) (layer "F.Cu") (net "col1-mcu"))
 (segment (start 194.92 73.424315) (end 194.92 80.555686) (width 0.2) (layer "F.Cu") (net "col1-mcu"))
 (segment (start 192.32 83.155686) (end 192.32 86.384314) (width 0.2) (layer "F.Cu") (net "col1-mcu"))
 (segment (start 194.105686 88.17) (end 198.14 88.17) (width 0.2) (layer "F.Cu") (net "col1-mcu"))
 (segment (start 192.32 86.384314) (end 194.105686 88.17) (width 0.2) (layer "F.Cu") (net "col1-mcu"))
 (segment (start 193.92 57.65) (end 193.92 72.424314) (width 0.2) (layer "F.Cu") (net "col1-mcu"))
 (segment (start 191.92 82.990001) (end 191.92 86.55) (width 0.2) (layer "F.Cu") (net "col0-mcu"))
 (segment (start 194.52 80.39) (end 191.92 82.990001) (width 0.2) (layer "F.Cu") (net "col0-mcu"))
 (segment (start 193.52 72.59) (end 194.52 73.59) (width 0.2) (layer "F.Cu") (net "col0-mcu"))
 (segment (start 193.52 59.79) (end 193.52 72.59) (width 0.2) (layer "F.Cu") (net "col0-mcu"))
 (segment (start 192.3 58.57) (end 193.52 59.79) (width 0.2) (layer "F.Cu") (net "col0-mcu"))
 (segment (start 194.52 73.59) (end 194.52 80.39) (width 0.2) (layer "F.Cu") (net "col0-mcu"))
 (segment (start 191.92 86.55) (end 194.04 88.67) (width 0.2) (layer "F.Cu") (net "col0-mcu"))
 (segment (start 194.04 88.67) (end 198.14 88.67) (width 0.2) (layer "F.Cu") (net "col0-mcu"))
 (segment (start 191.52 87.55) (end 193.64 89.67) (width 0.2) (layer "F.Cu") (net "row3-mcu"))
 (segment (start 191.52 69.51) (end 191.52 87.55) (width 0.2) (layer "F.Cu") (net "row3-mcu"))
 (segment (start 193.64 89.67) (end 197.64 89.67) (width 0.2) (layer "F.Cu") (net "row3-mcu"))
 (segment (start 192.3 68.73) (end 191.52 69.51) (width 0.2) (layer "F.Cu") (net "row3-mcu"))
 (segment (start 193.54 90.17) (end 197.64 90.17) (width 0.2) (layer "F.Cu") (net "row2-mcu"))
 (segment (start 192.3 66.19) (end 191.12 67.37) (width 0.2) (layer "F.Cu") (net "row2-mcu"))
 (segment (start 191.12 87.75) (end 193.54 90.17) (width 0.2) (layer "F.Cu") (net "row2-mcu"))
 (segment (start 191.12 67.37) (end 191.12 87.75) (width 0.2) (layer "F.Cu") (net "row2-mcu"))
 (segment (start 190.72 87.984314) (end 193.405686 90.67) (width 0.2) (layer "F.Cu") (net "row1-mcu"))
 (segment (start 192.3 63.65) (end 190.72 65.23) (width 0.2) (layer "F.Cu") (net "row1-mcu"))
 (segment (start 193.405686 90.67) (end 197.64 90.67) (width 0.2) (layer "F.Cu") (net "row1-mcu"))
 (segment (start 190.72 65.23) (end 190.72 87.984314) (width 0.2) (layer "F.Cu") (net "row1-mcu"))
 (segment (start 193.34 91.17) (end 197.64 91.17) (width 0.2) (layer "F.Cu") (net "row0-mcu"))
 (segment (start 192.3 61.11) (end 190.32 63.09) (width 0.2) (layer "F.Cu") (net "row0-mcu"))
 (segment (start 190.32 63.09) (end 190.32 88.15) (width 0.2) (layer "F.Cu") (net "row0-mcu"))
 (segment (start 190.32 88.15) (end 193.34 91.17) (width 0.2) (layer "F.Cu") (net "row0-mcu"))
 (segment (start 203.52 72.75) (end 207.54 68.73) (width 0.2) (layer "F.Cu") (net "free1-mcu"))
 (segment (start 197.64 91.67) (end 200.94 91.67) (width 0.2) (layer "F.Cu") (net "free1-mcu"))
 (segment (start 203.52 89.09) (end 203.52 72.75) (width 0.2) (layer "F.Cu") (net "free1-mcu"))
 (segment (start 200.94 91.67) (end 203.52 89.09) (width 0.2) (layer "F.Cu") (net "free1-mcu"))
 (segment (start 192.3 40.79) (end 197.3 40.79) (width 0.3) (layer "B.Cu") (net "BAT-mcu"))
 (segment (start 197.67 40.42) (end 197.67 40.22) (width 0.3) (layer "B.Cu") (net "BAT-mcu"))
 (segment (start 197.3 40.79) (end 197.67 40.42) (width 0.3) (layer "B.Cu") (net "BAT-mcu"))
 (segment (start 194.32 47.89) (end 194.32 49.59) (width 0.2) (layer "B.Cu") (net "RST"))
 (segment (start 194.32 49.59) (end 195.57 50.84) (width 0.2) (layer "B.Cu") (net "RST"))
 (segment (start 195.57 50.84) (end 196.82 50.84) (width 0.2) (layer "B.Cu") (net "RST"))
 (segment (start 196.82 50.84) (end 196.501802 50.521802) (width 0.2) (layer "B.Cu") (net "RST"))
 (segment (start 192.3 45.87) (end 194.32 47.89) (width 0.2) (layer "B.Cu") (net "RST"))
 (segment (start 196.82 50.84) (end 203.02 50.84) (width 0.2) (layer "B.Cu") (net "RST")))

